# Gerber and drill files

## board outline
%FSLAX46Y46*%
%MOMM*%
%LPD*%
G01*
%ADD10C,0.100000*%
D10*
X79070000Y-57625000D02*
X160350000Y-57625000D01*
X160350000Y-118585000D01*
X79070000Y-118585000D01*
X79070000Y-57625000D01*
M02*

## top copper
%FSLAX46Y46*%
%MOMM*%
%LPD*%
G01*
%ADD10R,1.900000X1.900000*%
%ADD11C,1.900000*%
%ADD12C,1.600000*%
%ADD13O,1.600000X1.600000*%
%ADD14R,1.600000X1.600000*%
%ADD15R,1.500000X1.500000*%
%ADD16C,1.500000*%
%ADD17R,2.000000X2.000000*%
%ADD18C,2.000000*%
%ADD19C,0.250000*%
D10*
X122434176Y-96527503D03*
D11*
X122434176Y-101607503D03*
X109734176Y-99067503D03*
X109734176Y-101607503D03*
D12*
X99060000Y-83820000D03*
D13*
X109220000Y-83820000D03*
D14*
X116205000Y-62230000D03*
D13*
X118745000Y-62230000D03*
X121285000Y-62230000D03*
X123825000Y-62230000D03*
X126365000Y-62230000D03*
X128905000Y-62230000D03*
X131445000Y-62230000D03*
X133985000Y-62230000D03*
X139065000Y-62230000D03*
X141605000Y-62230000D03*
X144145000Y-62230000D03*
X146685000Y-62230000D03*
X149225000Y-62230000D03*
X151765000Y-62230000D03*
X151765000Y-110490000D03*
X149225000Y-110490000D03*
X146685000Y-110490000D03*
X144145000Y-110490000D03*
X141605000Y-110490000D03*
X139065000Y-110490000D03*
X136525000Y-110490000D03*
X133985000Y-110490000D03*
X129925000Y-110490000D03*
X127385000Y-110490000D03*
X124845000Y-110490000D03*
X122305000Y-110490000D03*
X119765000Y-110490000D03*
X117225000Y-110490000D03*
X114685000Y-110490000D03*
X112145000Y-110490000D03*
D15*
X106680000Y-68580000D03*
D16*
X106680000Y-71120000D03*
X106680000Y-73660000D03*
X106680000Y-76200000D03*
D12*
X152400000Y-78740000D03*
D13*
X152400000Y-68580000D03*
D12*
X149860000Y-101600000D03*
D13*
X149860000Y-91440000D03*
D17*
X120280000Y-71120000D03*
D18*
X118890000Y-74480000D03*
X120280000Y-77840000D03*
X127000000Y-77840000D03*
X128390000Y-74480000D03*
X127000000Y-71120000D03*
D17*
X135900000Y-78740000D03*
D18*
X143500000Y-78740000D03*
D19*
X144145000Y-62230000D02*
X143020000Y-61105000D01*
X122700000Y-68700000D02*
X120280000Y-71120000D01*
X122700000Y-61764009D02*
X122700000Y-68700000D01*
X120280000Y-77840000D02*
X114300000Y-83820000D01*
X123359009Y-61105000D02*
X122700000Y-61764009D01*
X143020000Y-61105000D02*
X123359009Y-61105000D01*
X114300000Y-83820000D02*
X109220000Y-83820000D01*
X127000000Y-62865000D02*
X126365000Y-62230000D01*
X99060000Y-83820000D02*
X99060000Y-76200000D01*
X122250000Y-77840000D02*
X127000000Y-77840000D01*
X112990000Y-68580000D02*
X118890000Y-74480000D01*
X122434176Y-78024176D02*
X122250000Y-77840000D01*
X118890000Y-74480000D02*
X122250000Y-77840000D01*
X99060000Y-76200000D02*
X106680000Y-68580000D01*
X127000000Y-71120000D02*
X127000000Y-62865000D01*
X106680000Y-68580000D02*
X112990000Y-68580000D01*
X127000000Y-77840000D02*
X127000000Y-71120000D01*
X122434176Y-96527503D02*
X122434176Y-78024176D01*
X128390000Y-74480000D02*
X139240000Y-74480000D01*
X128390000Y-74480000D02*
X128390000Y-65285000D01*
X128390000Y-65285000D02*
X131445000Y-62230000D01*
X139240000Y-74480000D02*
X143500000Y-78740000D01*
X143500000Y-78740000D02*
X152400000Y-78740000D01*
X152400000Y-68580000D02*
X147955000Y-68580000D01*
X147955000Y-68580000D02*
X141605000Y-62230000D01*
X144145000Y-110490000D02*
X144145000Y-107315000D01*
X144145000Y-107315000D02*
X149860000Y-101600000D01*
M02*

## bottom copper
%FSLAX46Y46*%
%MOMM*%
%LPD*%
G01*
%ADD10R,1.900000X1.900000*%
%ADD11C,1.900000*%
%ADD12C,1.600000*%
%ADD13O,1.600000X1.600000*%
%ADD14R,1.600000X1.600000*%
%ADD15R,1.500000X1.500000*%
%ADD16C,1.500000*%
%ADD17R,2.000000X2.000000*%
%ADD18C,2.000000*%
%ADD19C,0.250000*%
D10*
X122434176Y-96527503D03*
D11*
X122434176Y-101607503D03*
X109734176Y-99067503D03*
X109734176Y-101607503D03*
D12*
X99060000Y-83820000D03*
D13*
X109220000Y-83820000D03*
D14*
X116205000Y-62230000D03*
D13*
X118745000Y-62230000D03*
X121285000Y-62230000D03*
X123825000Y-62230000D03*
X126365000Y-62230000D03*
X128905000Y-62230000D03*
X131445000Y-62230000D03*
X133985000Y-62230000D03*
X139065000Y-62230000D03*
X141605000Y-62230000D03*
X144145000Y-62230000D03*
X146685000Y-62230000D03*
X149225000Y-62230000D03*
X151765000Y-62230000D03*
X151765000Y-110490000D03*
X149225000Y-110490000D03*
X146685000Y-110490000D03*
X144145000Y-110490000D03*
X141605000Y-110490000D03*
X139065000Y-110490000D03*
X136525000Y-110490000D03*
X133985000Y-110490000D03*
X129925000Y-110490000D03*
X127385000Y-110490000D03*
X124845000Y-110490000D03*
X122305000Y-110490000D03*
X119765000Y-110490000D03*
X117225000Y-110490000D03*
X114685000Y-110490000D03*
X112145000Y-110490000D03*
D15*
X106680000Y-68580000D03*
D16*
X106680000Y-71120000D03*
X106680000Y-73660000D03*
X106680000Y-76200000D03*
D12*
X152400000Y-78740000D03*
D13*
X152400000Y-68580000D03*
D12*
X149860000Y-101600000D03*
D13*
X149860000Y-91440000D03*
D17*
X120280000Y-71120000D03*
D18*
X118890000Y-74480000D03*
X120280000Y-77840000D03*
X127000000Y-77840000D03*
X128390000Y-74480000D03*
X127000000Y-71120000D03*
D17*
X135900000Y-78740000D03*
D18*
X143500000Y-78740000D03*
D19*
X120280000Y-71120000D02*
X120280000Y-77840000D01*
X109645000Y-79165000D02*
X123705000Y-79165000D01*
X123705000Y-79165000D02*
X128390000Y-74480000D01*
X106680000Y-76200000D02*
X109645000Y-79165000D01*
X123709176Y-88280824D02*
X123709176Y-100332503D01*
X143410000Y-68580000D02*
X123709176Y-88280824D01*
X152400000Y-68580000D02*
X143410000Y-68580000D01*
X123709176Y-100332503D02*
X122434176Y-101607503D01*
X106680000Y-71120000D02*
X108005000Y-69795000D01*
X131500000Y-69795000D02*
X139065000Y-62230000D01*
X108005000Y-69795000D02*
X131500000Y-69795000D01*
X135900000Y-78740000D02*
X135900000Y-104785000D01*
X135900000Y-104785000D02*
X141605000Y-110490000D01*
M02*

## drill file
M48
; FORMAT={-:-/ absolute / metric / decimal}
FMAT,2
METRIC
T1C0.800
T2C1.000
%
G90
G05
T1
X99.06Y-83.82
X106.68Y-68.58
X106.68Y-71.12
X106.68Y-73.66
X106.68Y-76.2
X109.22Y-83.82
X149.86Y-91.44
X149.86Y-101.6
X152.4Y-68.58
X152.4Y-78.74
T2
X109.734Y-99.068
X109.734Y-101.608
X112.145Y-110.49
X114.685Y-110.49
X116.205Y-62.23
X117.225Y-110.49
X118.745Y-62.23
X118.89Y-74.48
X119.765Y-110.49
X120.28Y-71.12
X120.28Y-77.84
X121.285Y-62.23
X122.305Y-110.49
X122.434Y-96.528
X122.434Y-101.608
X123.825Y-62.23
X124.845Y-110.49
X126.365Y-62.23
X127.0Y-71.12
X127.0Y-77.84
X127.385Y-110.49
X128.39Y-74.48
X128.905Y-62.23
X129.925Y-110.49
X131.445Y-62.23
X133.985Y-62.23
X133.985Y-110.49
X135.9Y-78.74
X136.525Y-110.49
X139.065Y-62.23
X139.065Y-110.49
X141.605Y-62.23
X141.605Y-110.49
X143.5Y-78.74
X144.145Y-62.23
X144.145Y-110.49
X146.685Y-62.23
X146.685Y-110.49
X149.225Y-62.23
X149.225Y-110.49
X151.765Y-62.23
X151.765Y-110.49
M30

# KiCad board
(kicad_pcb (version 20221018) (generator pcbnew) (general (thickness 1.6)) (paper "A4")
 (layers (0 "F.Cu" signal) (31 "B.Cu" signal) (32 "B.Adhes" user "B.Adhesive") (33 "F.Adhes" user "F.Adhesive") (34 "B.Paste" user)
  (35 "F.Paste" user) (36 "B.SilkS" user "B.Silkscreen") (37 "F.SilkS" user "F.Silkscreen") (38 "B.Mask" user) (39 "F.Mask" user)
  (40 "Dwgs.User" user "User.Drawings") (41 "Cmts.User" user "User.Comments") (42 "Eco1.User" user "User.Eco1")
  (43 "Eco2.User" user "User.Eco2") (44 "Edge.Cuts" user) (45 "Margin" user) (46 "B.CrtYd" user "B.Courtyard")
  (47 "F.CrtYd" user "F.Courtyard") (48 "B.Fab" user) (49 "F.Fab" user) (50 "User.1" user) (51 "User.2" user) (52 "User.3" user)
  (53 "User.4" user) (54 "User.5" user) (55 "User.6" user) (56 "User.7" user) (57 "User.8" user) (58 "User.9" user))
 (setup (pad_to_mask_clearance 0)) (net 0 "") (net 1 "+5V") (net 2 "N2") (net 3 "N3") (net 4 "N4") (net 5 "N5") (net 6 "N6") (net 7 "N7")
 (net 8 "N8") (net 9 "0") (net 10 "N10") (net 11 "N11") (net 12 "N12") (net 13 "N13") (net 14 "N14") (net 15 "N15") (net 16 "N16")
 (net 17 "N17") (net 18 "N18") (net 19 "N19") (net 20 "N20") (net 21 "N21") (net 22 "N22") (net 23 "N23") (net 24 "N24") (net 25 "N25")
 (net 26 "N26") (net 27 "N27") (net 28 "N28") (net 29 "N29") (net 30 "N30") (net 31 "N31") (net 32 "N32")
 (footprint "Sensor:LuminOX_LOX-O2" (layer "F.Cu") (at 122.434176 96.527503)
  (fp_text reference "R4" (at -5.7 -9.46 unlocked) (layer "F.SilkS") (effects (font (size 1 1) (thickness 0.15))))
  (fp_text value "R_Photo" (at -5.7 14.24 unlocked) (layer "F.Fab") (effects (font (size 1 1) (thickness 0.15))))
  (pad "1" thru_hole rect (at 0 0) (size 1.9 1.9) (drill 1) (layers "*.Cu" "*.Mask") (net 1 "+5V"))
  (pad "2" thru_hole circle (at 0 5.08) (size 1.9 1.9) (drill 1) (layers "*.Cu" "*.Mask") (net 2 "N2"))
  (pad "3" thru_hole circle (at -12.7 2.54) (size 1.9 1.9) (drill 1) (layers "*.Cu" "*.Mask"))
  (pad "4" thru_hole circle (at -12.7 5.08) (size 1.9 1.9) (drill 1) (layers "*.Cu" "*.Mask")))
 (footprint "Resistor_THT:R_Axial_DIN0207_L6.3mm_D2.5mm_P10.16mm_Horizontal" (layer "F.Cu") (at 99.06 83.82)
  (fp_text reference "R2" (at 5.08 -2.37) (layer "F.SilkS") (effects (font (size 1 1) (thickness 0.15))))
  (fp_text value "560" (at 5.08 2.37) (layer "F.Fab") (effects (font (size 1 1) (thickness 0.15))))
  (pad "1" thru_hole circle (at 0 0) (size 1.6 1.6) (drill 0.8) (layers "*.Cu" "*.Mask") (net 1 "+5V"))
  (pad "2" thru_hole oval (at 10.16 0) (size 1.6 1.6) (drill 0.8) (layers "*.Cu" "*.Mask") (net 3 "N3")))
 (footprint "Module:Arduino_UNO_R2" (layer "F.Cu") (at 116.205 62.23)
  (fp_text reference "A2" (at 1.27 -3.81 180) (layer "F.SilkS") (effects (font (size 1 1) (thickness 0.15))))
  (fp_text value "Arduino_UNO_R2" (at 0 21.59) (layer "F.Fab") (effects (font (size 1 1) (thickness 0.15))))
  (pad "1" thru_hole rect (at 0 0 90) (size 1.6 1.6) (drill 1) (layers "*.Cu" "*.Mask") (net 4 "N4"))
  (pad "2" thru_hole oval (at 2.54 0 90) (size 1.6 1.6) (drill 1) (layers "*.Cu" "*.Mask") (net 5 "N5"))
  (pad "3" thru_hole oval (at 5.08 0 90) (size 1.6 1.6) (drill 1) (layers "*.Cu" "*.Mask") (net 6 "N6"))
  (pad "4" thru_hole oval (at 7.62 0 90) (size 1.6 1.6) (drill 1) (layers "*.Cu" "*.Mask") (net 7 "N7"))
  (pad "5" thru_hole oval (at 10.16 0 90) (size 1.6 1.6) (drill 1) (layers "*.Cu" "*.Mask") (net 1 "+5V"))
  (pad "6" thru_hole oval (at 12.7 0 90) (size 1.6 1.6) (drill 1) (layers "*.Cu" "*.Mask") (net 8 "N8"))
  (pad "7" thru_hole oval (at 15.24 0 90) (size 1.6 1.6) (drill 1) (layers "*.Cu" "*.Mask") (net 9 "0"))
  (pad "8" thru_hole oval (at 17.78 0 90) (size 1.6 1.6) (drill 1) (layers "*.Cu" "*.Mask") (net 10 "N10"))
  (pad "9" thru_hole oval (at 22.86 0 90) (size 1.6 1.6) (drill 1) (layers "*.Cu" "*.Mask") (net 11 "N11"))
  (pad "10" thru_hole oval (at 25.4 0 90) (size 1.6 1.6) (drill 1) (layers "*.Cu" "*.Mask") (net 2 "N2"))
  (pad "11" thru_hole oval (at 27.94 0 90) (size 1.6 1.6) (drill 1) (layers "*.Cu" "*.Mask") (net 3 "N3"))
  (pad "12" thru_hole oval (at 30.48 0 90) (size 1.6 1.6) (drill 1) (layers "*.Cu" "*.Mask") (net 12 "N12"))
  (pad "13" thru_hole oval (at 33.02 0 90) (size 1.6 1.6) (drill 1) (layers "*.Cu" "*.Mask") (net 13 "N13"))
  (pad "14" thru_hole oval (at 35.56 0 90) (size 1.6 1.6) (drill 1) (layers "*.Cu" "*.Mask") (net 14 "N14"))
  (pad "15" thru_hole oval (at 35.56 48.26 90) (size 1.6 1.6) (drill 1) (layers "*.Cu" "*.Mask") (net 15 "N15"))
  (pad "16" thru_hole oval (at 33.02 48.26 90) (size 1.6 1.6) (drill 1) (layers "*.Cu" "*.Mask") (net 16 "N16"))
  (pad "17" thru_hole oval (at 30.48 48.26 90) (size 1.6 1.6) (drill 1) (layers "*.Cu" "*.Mask") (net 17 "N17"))
  (pad "18" thru_hole oval (at 27.94 48.26 90) (size 1.6 1.6) (drill 1) (layers "*.Cu" "*.Mask") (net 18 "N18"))
  (pad "19" thru_hole oval (at 25.4 48.26 90) (size 1.6 1.6) (drill 1) (layers "*.Cu" "*.Mask") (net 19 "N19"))
  (pad "20" thru_hole oval (at 22.86 48.26 90) (size 1.6 1.6) (drill 1) (layers "*.Cu" "*.Mask") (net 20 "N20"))
  (pad "21" thru_hole oval (at 20.32 48.26 90) (size 1.6 1.6) (drill 1) (layers "*.Cu" "*.Mask") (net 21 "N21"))
  (pad "22" thru_hole oval (at 17.78 48.26 90) (size 1.6 1.6) (drill 1) (layers "*.Cu" "*.Mask") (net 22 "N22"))
  (pad "23" thru_hole oval (at 13.72 48.26 90) (size 1.6 1.6) (drill 1) (layers "*.Cu" "*.Mask") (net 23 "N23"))
  (pad "24" thru_hole oval (at 11.18 48.26 90) (size 1.6 1.6) (drill 1) (layers "*.Cu" "*.Mask") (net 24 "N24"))
  (pad "25" thru_hole oval (at 8.64 48.26 90) (size 1.6 1.6) (drill 1) (layers "*.Cu" "*.Mask") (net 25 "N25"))
  (pad "26" thru_hole oval (at 6.1 48.26 90) (size 1.6 1.6) (drill 1) (layers "*.Cu" "*.Mask") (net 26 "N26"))
  (pad "27" thru_hole oval (at 3.56 48.26 90) (size 1.6 1.6) (drill 1) (layers "*.Cu" "*.Mask") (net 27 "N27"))
  (pad "28" thru_hole oval (at 1.02 48.26 90) (size 1.6 1.6) (drill 1) (layers "*.Cu" "*.Mask") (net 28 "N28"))
  (pad "29" thru_hole oval (at -1.52 48.26 90) (size 1.6 1.6) (drill 1) (layers "*.Cu" "*.Mask") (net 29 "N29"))
  (pad "30" thru_hole oval (at -4.06 48.26 90) (size 1.6 1.6) (drill 1) (layers "*.Cu" "*.Mask") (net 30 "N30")))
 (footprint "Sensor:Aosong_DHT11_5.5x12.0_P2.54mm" (layer "F.Cu") (at 106.68 68.58)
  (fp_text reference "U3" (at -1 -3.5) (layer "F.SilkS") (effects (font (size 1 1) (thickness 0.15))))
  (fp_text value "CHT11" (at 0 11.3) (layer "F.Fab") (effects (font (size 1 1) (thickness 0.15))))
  (pad "1" thru_hole rect (at 0 0) (size 1.5 1.5) (drill 0.8) (layers "*.Cu" "*.Mask") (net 1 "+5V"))
  (pad "2" thru_hole circle (at 0 2.54) (size 1.5 1.5) (drill 0.8) (layers "*.Cu" "*.Mask") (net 11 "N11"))
  (pad "3" thru_hole circle (at 0 5.08) (size 1.5 1.5) (drill 0.8) (layers "*.Cu" "*.Mask") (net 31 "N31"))
  (pad "4" thru_hole circle (at 0 7.62) (size 1.5 1.5) (drill 0.8) (layers "*.Cu" "*.Mask") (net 9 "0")))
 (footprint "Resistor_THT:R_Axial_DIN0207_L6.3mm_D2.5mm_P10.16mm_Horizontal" (layer "F.Cu") (at 152.4 78.74 90)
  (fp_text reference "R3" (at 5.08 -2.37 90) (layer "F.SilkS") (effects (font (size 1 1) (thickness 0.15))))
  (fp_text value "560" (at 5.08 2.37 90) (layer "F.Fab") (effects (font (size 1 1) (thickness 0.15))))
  (pad "1" thru_hole circle (at 0 0 90) (size 1.6 1.6) (drill 0.8) (layers "*.Cu" "*.Mask") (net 9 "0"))
  (pad "2" thru_hole oval (at 10.16 0 90) (size 1.6 1.6) (drill 0.8) (layers "*.Cu" "*.Mask") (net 2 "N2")))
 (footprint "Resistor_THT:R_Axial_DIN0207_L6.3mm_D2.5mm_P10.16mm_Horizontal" (layer "F.Cu") (at 149.86 101.6 90)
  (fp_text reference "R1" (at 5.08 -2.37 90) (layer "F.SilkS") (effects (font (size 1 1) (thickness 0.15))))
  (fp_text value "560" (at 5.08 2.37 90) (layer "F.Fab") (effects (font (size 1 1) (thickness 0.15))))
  (pad "1" thru_hole circle (at 0 0 90) (size 1.6 1.6) (drill 0.8) (layers "*.Cu" "*.Mask") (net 18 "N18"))
  (pad "2" thru_hole oval (at 10.16 0 90) (size 1.6 1.6) (drill 0.8) (layers "*.Cu" "*.Mask") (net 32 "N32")))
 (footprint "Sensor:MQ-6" (layer "F.Cu") (at 120.28 71.12)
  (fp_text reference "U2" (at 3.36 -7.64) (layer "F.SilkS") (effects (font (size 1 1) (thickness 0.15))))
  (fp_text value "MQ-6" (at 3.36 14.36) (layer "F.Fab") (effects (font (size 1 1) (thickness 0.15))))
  (pad "1" thru_hole rect (at 0 0) (size 2 2) (drill 1) (layers "*.Cu" "*.Mask") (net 3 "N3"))
  (pad "2" thru_hole circle (at -1.39 3.36) (size 2 2) (drill 1) (layers "*.Cu" "*.Mask") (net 1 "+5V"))
  (pad "3" thru_hole circle (at 0 6.72 90) (size 2 2) (drill 1) (layers "*.Cu" "*.Mask") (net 3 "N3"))
  (pad "4" thru_hole circle (at 6.72 6.72 180) (size 2 2) (drill 1) (layers "*.Cu" "*.Mask") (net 1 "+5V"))
  (pad "5" thru_hole circle (at 8.11 3.36) (size 2 2) (drill 1) (layers "*.Cu" "*.Mask") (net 9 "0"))
  (pad "6" thru_hole circle (at 6.72 0 270) (size 2 2) (drill 1) (layers "*.Cu" "*.Mask") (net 1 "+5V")))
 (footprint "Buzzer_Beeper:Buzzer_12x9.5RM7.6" (layer "F.Cu") (at 135.9 78.74)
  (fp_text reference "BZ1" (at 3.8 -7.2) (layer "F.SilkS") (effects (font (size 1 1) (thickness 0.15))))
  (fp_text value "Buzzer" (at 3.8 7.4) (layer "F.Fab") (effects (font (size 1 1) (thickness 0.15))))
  (pad "1" thru_hole rect (at 0 0) (size 2 2) (drill 1) (layers "*.Cu" "*.Mask") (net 19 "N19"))
  (pad "2" thru_hole circle (at 7.6 0) (size 2 2) (drill 1) (layers "*.Cu" "*.Mask") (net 9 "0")))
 (gr_rect (start 79.07 57.625) (end 160.35 118.585) (stroke (width 0.1) (type default)) (fill none) (layer "Edge.Cuts"))
 (segment (start 144.145 62.23) (end 143.02 61.105) (width 0.25) (layer "F.Cu") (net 3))
 (segment (start 122.7 68.7) (end 120.28 71.12) (width 0.25) (layer "F.Cu") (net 3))
 (segment (start 122.7 61.764009) (end 122.7 68.7) (width 0.25) (layer "F.Cu") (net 3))
 (segment (start 120.28 77.84) (end 114.3 83.82) (width 0.25) (layer "F.Cu") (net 3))
 (segment (start 123.359009 61.105) (end 122.7 61.764009) (width 0.25) (layer "F.Cu") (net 3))
 (segment (start 143.02 61.105) (end 123.359009 61.105) (width 0.25) (layer "F.Cu") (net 3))
 (segment (start 114.3 83.82) (end 109.22 83.82) (width 0.25) (layer "F.Cu") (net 3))
 (segment (start 120.28 71.12) (end 120.28 77.84) (width 0.25) (layer "B.Cu") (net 3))
 (segment (start 127 62.865) (end 126.365 62.23) (width 0.25) (layer "F.Cu") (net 1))
 (segment (start 99.06 83.82) (end 99.06 76.2) (width 0.25) (layer "F.Cu") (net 1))
 (segment (start 122.25 77.84) (end 127 77.84) (width 0.25) (layer "F.Cu") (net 1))
 (segment (start 112.99 68.58) (end 118.89 74.48) (width 0.25) (layer "F.Cu") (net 1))
 (segment (start 122.434176 78.024176) (end 122.25 77.84) (width 0.25) (layer "F.Cu") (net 1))
 (segment (start 118.89 74.48) (end 122.25 77.84) (width 0.25) (layer "F.Cu") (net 1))
 (segment (start 99.06 76.2) (end 106.68 68.58) (width 0.25) (layer "F.Cu") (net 1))
 (segment (start 127 71.12) (end 127 62.865) (width 0.25) (layer "F.Cu") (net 1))
 (segment (start 106.68 68.58) (end 112.99 68.58) (width 0.25) (layer "F.Cu") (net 1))
 (segment (start 127 77.84) (end 127 71.12) (width 0.25) (layer "F.Cu") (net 1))
 (segment (start 122.434176 96.527503) (end 122.434176 78.024176) (width 0.25) (layer "F.Cu") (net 1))
 (segment (start 128.39 74.48) (end 139.24 74.48) (width 0.25) (layer "F.Cu") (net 9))
 (segment (start 128.39 74.48) (end 128.39 65.285) (width 0.25) (layer "F.Cu") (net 9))
 (segment (start 128.39 65.285) (end 131.445 62.23) (width 0.25) (layer "F.Cu") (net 9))
 (segment (start 139.24 74.48) (end 143.5 78.74) (width 0.25) (layer "F.Cu") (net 9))
 (segment (start 143.5 78.74) (end 152.4 78.74) (width 0.25) (layer "F.Cu") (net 9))
 (segment (start 109.645 79.165) (end 123.705 79.165) (width 0.25) (layer "B.Cu") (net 9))
 (segment (start 123.705 79.165) (end 128.39 74.48) (width 0.25) (layer "B.Cu") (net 9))
 (segment (start 106.68 76.2) (end 109.645 79.165) (width 0.25) (layer "B.Cu") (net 9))
 (segment (start 152.4 68.58) (end 147.955 68.58) (width 0.25) (layer "F.Cu") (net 2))
 (segment (start 147.955 68.58) (end 141.605 62.23) (width 0.25) (layer "F.Cu") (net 2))
 (segment (start 123.709176 88.280824) (end 123.709176 100.332503) (width 0.25) (layer "B.Cu") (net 2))
 (segment (start 143.41 68.58) (end 123.709176 88.280824) (width 0.25) (layer "B.Cu") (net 2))
 (segment (start 152.4 68.58) (end 143.41 68.58) (width 0.25) (layer "B.Cu") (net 2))
 (segment (start 123.709176 100.332503) (end 122.434176 101.607503) (width 0.25) (layer "B.Cu") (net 2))
 (segment (start 144.145 110.49) (end 144.145 107.315) (width 0.25) (layer "F.Cu") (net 18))
 (segment (start 144.145 107.315) (end 149.86 101.6) (width 0.25) (layer "F.Cu") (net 18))
 (segment (start 106.68 71.12) (end 108.005 69.795) (width 0.25) (layer "B.Cu") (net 11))
 (segment (start 131.5 69.795) (end 139.065 62.23) (width 0.25) (layer "B.Cu") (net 11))
 (segment (start 108.005 69.795) (end 131.5 69.795) (width 0.25) (layer "B.Cu") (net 11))
 (segment (start 135.9 78.74) (end 135.9 104.785) (width 0.25) (layer "B.Cu") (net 19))
 (segment (start 135.9 104.785) (end 141.605 110.49) (width 0.25) (layer "B.Cu") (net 19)))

